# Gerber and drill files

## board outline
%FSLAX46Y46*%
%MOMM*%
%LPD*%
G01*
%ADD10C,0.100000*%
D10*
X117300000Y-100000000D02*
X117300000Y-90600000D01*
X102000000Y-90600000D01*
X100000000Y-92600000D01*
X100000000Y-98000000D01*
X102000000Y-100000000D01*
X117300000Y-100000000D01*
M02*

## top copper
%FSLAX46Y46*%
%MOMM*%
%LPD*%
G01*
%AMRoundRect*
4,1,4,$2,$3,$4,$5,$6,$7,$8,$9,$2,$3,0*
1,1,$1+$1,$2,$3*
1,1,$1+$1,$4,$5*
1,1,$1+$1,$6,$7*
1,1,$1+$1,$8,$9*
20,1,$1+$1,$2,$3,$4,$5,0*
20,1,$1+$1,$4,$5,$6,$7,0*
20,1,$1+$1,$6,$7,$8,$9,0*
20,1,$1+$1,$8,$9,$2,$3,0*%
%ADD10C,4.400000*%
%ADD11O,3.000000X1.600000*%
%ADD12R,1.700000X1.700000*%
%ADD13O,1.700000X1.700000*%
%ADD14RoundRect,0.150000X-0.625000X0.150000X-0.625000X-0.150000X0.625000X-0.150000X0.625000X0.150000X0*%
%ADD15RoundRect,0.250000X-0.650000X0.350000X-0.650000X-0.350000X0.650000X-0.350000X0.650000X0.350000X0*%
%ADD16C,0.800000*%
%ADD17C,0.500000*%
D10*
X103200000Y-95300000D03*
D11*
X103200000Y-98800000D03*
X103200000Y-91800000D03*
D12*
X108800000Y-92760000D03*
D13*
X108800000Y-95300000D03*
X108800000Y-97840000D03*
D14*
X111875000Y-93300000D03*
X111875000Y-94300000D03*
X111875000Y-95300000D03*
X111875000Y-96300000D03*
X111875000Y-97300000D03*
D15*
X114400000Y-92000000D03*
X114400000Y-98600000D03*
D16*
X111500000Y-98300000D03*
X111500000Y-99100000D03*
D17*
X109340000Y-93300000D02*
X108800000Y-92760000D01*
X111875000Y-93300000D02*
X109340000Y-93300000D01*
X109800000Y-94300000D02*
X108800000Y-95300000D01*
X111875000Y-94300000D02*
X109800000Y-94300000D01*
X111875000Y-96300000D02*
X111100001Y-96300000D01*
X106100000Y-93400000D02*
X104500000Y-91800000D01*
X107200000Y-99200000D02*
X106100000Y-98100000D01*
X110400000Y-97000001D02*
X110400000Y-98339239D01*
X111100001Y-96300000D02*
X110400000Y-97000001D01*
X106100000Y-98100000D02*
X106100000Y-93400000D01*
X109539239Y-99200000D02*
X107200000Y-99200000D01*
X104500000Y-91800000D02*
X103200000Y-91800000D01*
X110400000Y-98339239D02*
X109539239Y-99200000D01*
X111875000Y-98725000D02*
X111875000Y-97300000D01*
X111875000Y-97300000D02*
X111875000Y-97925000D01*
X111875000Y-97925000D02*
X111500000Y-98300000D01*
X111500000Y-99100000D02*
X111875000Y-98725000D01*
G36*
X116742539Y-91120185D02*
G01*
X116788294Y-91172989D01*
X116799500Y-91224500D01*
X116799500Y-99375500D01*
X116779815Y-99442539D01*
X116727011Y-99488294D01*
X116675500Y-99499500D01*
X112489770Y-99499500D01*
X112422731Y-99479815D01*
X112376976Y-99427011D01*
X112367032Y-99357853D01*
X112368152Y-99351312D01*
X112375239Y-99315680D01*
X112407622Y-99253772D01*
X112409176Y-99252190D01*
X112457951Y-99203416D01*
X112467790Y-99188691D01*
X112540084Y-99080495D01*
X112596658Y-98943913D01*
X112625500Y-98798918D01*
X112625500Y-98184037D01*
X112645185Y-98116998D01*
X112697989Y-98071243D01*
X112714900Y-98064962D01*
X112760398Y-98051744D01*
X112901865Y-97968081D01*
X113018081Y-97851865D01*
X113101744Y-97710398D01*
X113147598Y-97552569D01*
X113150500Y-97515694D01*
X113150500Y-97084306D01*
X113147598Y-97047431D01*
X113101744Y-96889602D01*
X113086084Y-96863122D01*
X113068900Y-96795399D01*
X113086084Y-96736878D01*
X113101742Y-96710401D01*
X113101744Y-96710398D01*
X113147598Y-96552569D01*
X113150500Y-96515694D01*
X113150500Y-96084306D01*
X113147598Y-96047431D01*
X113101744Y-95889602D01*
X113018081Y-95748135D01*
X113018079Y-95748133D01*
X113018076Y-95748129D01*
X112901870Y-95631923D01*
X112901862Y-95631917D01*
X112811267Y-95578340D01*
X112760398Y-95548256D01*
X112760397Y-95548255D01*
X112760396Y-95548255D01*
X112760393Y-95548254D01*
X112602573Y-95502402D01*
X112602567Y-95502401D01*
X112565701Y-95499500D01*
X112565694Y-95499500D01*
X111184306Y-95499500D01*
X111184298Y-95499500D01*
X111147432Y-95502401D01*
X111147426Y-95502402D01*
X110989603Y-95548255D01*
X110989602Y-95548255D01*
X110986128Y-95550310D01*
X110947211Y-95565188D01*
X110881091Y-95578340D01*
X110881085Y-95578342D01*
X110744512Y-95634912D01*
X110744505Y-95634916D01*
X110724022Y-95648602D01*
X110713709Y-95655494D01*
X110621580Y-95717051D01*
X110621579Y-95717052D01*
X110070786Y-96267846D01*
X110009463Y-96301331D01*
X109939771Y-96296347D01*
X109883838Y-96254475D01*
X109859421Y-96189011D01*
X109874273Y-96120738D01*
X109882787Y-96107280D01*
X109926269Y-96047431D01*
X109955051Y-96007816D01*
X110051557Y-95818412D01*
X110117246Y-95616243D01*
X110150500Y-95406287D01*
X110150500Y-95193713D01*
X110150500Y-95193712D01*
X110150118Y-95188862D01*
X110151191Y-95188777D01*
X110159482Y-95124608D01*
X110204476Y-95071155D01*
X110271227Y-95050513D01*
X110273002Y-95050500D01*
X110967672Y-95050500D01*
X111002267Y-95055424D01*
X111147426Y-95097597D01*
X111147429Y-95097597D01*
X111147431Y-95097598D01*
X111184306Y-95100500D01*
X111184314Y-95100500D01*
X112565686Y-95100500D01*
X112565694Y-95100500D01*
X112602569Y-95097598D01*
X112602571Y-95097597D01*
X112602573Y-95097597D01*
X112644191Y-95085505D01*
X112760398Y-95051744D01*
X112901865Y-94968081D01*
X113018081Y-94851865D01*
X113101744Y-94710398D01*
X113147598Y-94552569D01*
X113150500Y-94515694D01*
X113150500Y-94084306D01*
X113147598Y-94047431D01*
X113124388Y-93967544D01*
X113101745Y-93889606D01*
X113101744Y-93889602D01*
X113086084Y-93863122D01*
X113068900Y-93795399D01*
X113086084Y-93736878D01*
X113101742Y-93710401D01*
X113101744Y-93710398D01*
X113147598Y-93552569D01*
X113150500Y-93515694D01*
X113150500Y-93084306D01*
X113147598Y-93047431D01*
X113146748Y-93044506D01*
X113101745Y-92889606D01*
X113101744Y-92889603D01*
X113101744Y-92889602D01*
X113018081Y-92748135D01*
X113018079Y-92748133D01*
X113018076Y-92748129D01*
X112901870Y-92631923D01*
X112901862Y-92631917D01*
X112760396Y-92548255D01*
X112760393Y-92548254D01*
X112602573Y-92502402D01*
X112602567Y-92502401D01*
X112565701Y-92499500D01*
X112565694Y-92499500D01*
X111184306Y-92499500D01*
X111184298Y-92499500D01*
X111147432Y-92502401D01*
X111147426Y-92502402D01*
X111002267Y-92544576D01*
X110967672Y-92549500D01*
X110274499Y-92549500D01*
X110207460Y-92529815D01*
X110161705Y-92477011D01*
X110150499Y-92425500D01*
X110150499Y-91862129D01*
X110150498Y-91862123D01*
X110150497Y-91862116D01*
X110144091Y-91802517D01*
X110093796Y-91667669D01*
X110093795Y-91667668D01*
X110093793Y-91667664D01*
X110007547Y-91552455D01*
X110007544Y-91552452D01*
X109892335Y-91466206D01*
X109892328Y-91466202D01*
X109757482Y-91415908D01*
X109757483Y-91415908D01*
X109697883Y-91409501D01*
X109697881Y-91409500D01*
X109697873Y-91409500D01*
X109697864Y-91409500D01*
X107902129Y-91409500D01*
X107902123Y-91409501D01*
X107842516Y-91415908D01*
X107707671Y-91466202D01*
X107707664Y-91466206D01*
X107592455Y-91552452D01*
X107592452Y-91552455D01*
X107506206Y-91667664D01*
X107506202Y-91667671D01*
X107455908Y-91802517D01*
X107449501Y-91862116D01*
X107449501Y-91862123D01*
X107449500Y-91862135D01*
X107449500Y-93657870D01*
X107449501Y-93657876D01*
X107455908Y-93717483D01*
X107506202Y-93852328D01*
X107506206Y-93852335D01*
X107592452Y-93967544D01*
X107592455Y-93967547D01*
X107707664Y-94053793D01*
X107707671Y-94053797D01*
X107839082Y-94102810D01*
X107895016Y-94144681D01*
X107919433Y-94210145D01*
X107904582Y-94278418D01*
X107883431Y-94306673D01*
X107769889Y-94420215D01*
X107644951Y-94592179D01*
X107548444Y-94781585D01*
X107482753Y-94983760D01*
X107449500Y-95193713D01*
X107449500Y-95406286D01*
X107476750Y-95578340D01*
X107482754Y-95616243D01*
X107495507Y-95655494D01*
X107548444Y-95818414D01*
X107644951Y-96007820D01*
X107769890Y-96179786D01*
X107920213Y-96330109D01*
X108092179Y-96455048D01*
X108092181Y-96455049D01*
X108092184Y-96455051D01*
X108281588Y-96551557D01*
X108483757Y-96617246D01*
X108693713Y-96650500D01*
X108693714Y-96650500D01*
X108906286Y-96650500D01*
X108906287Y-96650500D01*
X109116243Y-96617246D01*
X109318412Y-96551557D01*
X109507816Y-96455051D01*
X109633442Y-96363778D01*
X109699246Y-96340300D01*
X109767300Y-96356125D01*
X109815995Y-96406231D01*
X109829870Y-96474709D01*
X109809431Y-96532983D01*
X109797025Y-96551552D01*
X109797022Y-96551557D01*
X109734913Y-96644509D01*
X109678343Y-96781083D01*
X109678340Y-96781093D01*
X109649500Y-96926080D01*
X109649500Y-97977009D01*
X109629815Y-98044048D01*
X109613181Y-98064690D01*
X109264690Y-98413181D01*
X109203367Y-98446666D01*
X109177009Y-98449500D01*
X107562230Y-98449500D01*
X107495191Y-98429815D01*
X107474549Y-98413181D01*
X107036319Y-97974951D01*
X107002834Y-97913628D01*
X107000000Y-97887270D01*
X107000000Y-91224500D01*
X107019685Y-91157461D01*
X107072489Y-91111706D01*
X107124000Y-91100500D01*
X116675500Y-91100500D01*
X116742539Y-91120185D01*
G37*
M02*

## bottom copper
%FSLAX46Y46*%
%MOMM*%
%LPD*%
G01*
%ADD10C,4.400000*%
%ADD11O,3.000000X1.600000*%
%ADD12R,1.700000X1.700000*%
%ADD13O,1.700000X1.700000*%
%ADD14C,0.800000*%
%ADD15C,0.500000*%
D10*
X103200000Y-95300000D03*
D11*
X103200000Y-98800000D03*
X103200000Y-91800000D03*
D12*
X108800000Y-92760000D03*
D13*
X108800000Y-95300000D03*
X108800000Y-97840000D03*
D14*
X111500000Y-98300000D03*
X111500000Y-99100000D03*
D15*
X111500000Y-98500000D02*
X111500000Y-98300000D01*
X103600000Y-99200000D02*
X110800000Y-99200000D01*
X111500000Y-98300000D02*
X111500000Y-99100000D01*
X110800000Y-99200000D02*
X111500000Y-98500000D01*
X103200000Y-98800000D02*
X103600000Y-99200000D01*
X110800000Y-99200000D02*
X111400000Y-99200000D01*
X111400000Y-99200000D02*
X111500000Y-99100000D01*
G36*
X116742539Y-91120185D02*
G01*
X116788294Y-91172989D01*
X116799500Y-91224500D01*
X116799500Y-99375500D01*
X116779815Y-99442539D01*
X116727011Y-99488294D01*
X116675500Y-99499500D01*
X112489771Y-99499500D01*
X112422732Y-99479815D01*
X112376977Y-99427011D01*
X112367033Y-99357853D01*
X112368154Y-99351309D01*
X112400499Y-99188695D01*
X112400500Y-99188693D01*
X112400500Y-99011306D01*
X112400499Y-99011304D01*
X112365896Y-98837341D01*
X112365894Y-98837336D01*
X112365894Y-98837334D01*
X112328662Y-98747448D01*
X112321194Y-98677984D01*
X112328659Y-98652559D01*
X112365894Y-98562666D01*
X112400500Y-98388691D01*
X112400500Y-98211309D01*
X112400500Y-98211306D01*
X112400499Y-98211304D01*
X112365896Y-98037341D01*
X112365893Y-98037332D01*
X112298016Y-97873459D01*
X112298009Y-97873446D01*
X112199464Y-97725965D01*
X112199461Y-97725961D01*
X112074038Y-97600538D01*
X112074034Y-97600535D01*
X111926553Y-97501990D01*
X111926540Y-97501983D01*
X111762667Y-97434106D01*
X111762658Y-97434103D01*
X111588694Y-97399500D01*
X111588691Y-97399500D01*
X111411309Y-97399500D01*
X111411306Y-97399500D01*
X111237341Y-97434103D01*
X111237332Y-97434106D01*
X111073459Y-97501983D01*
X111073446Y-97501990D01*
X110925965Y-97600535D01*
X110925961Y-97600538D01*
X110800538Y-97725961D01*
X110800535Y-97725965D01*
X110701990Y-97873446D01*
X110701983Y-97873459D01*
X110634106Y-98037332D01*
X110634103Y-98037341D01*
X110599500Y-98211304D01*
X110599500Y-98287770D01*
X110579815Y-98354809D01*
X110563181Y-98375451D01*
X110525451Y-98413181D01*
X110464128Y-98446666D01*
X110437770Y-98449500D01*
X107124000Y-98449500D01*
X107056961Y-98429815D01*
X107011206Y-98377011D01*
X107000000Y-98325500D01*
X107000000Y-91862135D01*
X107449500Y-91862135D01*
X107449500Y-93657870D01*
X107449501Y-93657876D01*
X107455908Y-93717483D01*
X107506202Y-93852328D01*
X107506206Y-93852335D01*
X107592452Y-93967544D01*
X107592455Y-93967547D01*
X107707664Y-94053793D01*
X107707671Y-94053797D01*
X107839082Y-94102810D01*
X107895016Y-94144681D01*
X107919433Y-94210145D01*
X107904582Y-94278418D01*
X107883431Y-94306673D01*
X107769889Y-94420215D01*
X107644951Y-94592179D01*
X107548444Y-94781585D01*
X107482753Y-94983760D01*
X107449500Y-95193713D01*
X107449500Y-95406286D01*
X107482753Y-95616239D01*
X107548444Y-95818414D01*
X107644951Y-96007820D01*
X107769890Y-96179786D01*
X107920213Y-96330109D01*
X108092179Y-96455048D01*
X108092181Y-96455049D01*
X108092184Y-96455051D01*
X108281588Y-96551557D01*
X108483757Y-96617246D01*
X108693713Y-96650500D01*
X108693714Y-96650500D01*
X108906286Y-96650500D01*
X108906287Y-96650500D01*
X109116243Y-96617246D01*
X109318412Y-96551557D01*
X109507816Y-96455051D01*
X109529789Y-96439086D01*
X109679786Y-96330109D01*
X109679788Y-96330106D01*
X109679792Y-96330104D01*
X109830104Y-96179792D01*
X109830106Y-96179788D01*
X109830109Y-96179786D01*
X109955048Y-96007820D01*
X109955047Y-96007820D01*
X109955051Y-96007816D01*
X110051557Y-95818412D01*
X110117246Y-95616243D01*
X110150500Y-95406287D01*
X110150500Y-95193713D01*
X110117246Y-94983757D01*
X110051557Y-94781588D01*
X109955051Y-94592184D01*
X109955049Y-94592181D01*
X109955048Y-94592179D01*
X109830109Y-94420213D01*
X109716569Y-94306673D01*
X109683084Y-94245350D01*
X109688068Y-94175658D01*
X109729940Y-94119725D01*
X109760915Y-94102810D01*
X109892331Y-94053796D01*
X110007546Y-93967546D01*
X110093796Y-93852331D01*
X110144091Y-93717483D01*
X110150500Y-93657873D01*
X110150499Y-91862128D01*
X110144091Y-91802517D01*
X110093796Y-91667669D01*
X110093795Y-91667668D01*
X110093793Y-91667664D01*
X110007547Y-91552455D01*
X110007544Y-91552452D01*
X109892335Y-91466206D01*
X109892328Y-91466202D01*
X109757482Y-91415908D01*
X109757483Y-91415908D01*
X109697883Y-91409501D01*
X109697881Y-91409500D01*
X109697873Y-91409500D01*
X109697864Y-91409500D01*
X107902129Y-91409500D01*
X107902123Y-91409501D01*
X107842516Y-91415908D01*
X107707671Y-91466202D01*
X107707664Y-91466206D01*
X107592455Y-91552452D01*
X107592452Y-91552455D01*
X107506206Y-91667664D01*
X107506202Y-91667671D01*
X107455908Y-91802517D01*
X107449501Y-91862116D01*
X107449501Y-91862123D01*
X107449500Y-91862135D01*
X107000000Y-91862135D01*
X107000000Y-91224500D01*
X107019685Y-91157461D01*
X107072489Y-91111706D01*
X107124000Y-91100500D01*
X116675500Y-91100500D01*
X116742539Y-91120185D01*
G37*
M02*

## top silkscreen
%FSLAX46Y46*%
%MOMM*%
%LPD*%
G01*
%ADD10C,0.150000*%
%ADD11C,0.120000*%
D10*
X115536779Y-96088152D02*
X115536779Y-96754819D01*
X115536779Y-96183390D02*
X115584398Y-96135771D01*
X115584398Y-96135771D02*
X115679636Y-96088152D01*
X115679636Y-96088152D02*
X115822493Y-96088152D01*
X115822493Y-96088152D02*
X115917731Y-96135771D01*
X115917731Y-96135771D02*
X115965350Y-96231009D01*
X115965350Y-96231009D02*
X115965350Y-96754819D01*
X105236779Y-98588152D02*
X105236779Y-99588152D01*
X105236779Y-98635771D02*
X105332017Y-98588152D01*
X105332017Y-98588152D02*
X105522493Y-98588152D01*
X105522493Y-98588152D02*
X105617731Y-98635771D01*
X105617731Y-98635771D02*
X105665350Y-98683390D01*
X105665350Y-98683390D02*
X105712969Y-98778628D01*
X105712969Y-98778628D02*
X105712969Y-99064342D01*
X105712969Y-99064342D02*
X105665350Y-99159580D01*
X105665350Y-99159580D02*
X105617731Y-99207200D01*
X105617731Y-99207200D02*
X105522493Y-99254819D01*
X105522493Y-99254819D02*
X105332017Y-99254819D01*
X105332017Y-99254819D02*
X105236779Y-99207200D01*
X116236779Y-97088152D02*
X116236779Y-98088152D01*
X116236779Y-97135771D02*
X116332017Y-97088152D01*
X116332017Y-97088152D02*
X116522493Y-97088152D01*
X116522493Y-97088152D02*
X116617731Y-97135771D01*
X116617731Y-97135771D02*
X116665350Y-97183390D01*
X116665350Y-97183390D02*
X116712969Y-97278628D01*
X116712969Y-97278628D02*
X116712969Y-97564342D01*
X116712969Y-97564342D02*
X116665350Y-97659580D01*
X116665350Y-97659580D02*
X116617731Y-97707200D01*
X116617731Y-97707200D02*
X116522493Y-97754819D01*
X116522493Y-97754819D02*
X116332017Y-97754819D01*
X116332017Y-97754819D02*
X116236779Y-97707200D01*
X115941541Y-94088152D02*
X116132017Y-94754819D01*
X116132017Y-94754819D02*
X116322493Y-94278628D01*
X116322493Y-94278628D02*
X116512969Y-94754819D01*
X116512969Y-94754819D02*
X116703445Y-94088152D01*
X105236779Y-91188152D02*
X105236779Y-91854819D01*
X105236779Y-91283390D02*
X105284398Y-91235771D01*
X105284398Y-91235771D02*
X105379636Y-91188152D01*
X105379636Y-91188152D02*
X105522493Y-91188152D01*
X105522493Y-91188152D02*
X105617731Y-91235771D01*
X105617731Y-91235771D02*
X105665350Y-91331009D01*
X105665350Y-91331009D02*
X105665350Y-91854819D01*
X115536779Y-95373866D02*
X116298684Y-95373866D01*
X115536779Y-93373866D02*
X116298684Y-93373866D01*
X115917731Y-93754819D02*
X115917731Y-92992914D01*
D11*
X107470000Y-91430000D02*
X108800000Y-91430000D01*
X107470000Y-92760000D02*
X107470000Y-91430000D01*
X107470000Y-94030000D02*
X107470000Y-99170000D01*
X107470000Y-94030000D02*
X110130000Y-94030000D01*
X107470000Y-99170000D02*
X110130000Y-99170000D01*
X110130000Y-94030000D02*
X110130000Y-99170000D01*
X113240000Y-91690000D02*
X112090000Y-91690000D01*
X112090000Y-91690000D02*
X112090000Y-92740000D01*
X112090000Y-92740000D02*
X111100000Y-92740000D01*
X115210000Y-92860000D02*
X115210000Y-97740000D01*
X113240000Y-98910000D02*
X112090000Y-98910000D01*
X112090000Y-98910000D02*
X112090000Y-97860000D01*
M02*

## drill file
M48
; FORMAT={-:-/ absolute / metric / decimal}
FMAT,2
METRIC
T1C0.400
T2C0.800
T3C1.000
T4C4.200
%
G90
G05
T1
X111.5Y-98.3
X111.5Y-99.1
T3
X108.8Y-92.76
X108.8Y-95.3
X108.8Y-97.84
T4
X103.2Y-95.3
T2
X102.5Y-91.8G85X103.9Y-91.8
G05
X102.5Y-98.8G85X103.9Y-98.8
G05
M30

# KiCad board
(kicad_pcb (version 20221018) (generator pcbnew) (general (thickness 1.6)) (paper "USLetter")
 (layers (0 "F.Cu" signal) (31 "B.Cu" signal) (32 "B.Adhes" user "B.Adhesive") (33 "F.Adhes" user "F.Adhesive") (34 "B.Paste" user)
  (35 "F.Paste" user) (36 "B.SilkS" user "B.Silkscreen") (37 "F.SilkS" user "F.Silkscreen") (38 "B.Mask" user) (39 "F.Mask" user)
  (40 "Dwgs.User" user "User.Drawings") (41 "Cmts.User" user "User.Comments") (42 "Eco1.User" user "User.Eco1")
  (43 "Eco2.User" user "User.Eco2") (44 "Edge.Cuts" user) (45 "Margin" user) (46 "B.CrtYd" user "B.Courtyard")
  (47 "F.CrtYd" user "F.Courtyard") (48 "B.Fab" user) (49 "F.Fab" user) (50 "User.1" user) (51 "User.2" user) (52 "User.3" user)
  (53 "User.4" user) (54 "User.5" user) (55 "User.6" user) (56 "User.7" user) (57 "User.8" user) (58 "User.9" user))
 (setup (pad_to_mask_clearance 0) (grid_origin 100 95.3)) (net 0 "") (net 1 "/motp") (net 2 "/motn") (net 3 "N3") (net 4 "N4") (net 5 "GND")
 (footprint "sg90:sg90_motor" (layer "F.Cu") (at 103.2 95.3)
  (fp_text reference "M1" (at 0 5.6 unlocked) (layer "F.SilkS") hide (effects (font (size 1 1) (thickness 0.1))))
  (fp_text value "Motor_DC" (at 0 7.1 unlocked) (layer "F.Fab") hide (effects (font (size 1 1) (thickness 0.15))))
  (pad "" thru_hole circle (at 0 0) (size 4.4 4.4) (drill 4.2) (layers "*.Cu" "*.Mask"))
  (pad "1" thru_hole oval (at 0 3.5) (size 3 1.6) (drill oval 2.2 0.8) (layers "*.Cu" "*.Mask") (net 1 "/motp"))
  (pad "2" thru_hole oval (at 0 -3.5) (size 3 1.6) (drill oval 2.2 0.8) (layers "*.Cu" "*.Mask") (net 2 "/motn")))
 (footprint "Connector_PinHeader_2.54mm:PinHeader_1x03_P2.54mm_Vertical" (layer "F.Cu") (at 108.8 92.76)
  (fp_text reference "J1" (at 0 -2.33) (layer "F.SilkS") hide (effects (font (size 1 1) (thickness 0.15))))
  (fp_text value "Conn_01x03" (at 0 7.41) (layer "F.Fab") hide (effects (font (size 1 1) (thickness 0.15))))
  (fp_line (start -1.33 -1.33) (end 0 -1.33) (stroke (width 0.12) (type solid)) (layer "F.SilkS"))
  (fp_line (start -1.33 0) (end -1.33 -1.33) (stroke (width 0.12) (type solid)) (layer "F.SilkS"))
  (fp_line (start -1.33 1.27) (end -1.33 6.41) (stroke (width 0.12) (type solid)) (layer "F.SilkS"))
  (fp_line (start -1.33 1.27) (end 1.33 1.27) (stroke (width 0.12) (type solid)) (layer "F.SilkS"))
  (fp_line (start -1.33 6.41) (end 1.33 6.41) (stroke (width 0.12) (type solid)) (layer "F.SilkS"))
  (fp_line (start 1.33 1.27) (end 1.33 6.41) (stroke (width 0.12) (type solid)) (layer "F.SilkS"))
  (pad "1" thru_hole rect (at 0 0) (size 1.7 1.7) (drill 1) (layers "*.Cu" "*.Mask") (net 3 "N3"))
  (pad "2" thru_hole oval (at 0 2.54) (size 1.7 1.7) (drill 1) (layers "*.Cu" "*.Mask") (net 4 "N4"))
  (pad "3" thru_hole oval (at 0 5.08) (size 1.7 1.7) (drill 1) (layers "*.Cu" "*.Mask") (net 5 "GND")))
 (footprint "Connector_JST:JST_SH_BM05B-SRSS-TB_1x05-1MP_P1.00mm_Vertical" (layer "F.Cu") (at 113.2 95.3 -90)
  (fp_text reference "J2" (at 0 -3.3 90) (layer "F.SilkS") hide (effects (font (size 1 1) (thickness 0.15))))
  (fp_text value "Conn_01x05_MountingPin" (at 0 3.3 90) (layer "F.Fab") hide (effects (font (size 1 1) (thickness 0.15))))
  (fp_line (start -3.61 -0.04) (end -3.61 1.11) (stroke (width 0.12) (type solid)) (layer "F.SilkS"))
  (fp_line (start -3.61 1.11) (end -2.56 1.11) (stroke (width 0.12) (type solid)) (layer "F.SilkS"))
  (fp_line (start -2.56 1.11) (end -2.56 2.1) (stroke (width 0.12) (type solid)) (layer "F.SilkS"))
  (fp_line (start -2.44 -2.01) (end 2.44 -2.01) (stroke (width 0.12) (type solid)) (layer "F.SilkS"))
  (fp_line (start 3.61 -0.04) (end 3.61 1.11) (stroke (width 0.12) (type solid)) (layer "F.SilkS"))
  (fp_line (start 3.61 1.11) (end 2.56 1.11) (stroke (width 0.12) (type solid)) (layer "F.SilkS"))
  (pad "1" smd roundrect (at -2 1.325 270) (size 0.6 1.55) (layers "F.Cu" "F.Paste" "F.Mask") (roundrect_rratio 0.25) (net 3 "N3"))
  (pad "2" smd roundrect (at -1 1.325 270) (size 0.6 1.55) (layers "F.Cu" "F.Paste" "F.Mask") (roundrect_rratio 0.25) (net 4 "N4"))
  (pad "3" smd roundrect (at 0 1.325 270) (size 0.6 1.55) (layers "F.Cu" "F.Paste" "F.Mask") (roundrect_rratio 0.25) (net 5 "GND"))
  (pad "4" smd roundrect (at 1 1.325 270) (size 0.6 1.55) (layers "F.Cu" "F.Paste" "F.Mask") (roundrect_rratio 0.25) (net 2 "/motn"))
  (pad "5" smd roundrect (at 2 1.325 270) (size 0.6 1.55) (layers "F.Cu" "F.Paste" "F.Mask") (roundrect_rratio 0.25) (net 1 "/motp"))
  (pad "MP" smd roundrect (at -3.3 -1.2 270) (size 1.2 1.8) (layers "F.Cu" "F.Paste" "F.Mask") (roundrect_rratio 0.208333) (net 5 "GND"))
  (pad "MP" smd roundrect (at 3.3 -1.2 270) (size 1.2 1.8) (layers "F.Cu" "F.Paste" "F.Mask") (roundrect_rratio 0.208333) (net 5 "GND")))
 (gr_poly
  (pts (xy 117.3 100) (xy 117.3 90.6) (xy 102 90.6) (xy 100 92.6) (xy 100 98) (xy 102 100)) (stroke (width 0.1) (type solid)) (fill none)
  (layer "Edge.Cuts"))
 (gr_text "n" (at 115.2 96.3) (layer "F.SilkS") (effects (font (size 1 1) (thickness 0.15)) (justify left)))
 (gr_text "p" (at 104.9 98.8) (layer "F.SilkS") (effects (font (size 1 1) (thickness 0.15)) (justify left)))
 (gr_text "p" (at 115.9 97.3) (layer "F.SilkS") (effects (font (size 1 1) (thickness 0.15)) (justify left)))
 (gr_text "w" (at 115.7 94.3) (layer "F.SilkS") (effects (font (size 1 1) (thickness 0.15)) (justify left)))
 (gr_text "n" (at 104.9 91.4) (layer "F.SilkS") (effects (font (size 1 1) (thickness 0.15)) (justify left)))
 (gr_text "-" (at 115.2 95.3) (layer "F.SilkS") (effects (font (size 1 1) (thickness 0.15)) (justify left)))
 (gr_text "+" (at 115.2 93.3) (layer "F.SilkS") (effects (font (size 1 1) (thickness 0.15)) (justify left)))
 (segment (start 109.34 93.3) (end 108.8 92.76) (width 0.5) (layer "F.Cu") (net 3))
 (segment (start 111.875 93.3) (end 109.34 93.3) (width 0.5) (layer "F.Cu") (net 3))
 (segment (start 109.8 94.3) (end 108.8 95.3) (width 0.5) (layer "F.Cu") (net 4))
 (segment (start 111.875 94.3) (end 109.8 94.3) (width 0.5) (layer "F.Cu") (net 4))
 (segment (start 111.875 96.3) (end 111.100001 96.3) (width 0.5) (layer "F.Cu") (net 2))
 (segment (start 106.1 93.4) (end 104.5 91.8) (width 0.5) (layer "F.Cu") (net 2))
 (segment (start 107.2 99.2) (end 106.1 98.1) (width 0.5) (layer "F.Cu") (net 2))
 (segment (start 110.4 97.000001) (end 110.4 98.339239) (width 0.5) (layer "F.Cu") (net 2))
 (segment (start 111.100001 96.3) (end 110.4 97.000001) (width 0.5) (layer "F.Cu") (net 2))
 (segment (start 106.1 98.1) (end 106.1 93.4) (width 0.5) (layer "F.Cu") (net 2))
 (segment (start 109.539239 99.2) (end 107.2 99.2) (width 0.5) (layer "F.Cu") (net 2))
 (segment (start 104.5 91.8) (end 103.2 91.8) (width 0.5) (layer "F.Cu") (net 2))
 (segment (start 110.4 98.339239) (end 109.539239 99.2) (width 0.5) (layer "F.Cu") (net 2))
 (segment (start 111.875 98.725) (end 111.875 97.3) (width 0.5) (layer "F.Cu") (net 1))
 (segment (start 111.875 97.3) (end 111.875 97.925) (width 0.5) (layer "F.Cu") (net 1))
 (segment (start 111.875 97.925) (end 111.5 98.3) (width 0.5) (layer "F.Cu") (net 1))
 (segment (start 111.5 99.1) (end 111.875 98.725) (width 0.5) (layer "F.Cu") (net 1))
 (via (at 111.5 98.3) (size 0.8) (drill 0.4) (layers "F.Cu" "B.Cu") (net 1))
 (via (at 111.5 99.1) (size 0.8) (drill 0.4) (layers "F.Cu" "B.Cu") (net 1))
 (segment (start 111.5 98.5) (end 111.5 98.3) (width 0.5) (layer "B.Cu") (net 1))
 (segment (start 103.6 99.2) (end 110.8 99.2) (width 0.5) (layer "B.Cu") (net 1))
 (segment (start 111.5 98.3) (end 111.5 99.1) (width 0.5) (layer "B.Cu") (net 1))
 (segment (start 110.8 99.2) (end 111.5 98.5) (width 0.5) (layer "B.Cu") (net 1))
 (segment (start 103.2 98.8) (end 103.6 99.2) (width 0.5) (layer "B.Cu") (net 1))
 (segment (start 110.8 99.2) (end 111.4 99.2) (width 0.5) (layer "B.Cu") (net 1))
 (segment (start 111.4 99.2) (end 111.5 99.1) (width 0.5) (layer "B.Cu") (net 1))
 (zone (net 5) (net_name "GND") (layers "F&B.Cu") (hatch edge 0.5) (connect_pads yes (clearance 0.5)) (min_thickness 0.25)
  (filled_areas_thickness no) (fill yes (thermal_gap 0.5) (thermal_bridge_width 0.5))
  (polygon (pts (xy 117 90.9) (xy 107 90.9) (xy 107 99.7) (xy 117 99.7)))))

